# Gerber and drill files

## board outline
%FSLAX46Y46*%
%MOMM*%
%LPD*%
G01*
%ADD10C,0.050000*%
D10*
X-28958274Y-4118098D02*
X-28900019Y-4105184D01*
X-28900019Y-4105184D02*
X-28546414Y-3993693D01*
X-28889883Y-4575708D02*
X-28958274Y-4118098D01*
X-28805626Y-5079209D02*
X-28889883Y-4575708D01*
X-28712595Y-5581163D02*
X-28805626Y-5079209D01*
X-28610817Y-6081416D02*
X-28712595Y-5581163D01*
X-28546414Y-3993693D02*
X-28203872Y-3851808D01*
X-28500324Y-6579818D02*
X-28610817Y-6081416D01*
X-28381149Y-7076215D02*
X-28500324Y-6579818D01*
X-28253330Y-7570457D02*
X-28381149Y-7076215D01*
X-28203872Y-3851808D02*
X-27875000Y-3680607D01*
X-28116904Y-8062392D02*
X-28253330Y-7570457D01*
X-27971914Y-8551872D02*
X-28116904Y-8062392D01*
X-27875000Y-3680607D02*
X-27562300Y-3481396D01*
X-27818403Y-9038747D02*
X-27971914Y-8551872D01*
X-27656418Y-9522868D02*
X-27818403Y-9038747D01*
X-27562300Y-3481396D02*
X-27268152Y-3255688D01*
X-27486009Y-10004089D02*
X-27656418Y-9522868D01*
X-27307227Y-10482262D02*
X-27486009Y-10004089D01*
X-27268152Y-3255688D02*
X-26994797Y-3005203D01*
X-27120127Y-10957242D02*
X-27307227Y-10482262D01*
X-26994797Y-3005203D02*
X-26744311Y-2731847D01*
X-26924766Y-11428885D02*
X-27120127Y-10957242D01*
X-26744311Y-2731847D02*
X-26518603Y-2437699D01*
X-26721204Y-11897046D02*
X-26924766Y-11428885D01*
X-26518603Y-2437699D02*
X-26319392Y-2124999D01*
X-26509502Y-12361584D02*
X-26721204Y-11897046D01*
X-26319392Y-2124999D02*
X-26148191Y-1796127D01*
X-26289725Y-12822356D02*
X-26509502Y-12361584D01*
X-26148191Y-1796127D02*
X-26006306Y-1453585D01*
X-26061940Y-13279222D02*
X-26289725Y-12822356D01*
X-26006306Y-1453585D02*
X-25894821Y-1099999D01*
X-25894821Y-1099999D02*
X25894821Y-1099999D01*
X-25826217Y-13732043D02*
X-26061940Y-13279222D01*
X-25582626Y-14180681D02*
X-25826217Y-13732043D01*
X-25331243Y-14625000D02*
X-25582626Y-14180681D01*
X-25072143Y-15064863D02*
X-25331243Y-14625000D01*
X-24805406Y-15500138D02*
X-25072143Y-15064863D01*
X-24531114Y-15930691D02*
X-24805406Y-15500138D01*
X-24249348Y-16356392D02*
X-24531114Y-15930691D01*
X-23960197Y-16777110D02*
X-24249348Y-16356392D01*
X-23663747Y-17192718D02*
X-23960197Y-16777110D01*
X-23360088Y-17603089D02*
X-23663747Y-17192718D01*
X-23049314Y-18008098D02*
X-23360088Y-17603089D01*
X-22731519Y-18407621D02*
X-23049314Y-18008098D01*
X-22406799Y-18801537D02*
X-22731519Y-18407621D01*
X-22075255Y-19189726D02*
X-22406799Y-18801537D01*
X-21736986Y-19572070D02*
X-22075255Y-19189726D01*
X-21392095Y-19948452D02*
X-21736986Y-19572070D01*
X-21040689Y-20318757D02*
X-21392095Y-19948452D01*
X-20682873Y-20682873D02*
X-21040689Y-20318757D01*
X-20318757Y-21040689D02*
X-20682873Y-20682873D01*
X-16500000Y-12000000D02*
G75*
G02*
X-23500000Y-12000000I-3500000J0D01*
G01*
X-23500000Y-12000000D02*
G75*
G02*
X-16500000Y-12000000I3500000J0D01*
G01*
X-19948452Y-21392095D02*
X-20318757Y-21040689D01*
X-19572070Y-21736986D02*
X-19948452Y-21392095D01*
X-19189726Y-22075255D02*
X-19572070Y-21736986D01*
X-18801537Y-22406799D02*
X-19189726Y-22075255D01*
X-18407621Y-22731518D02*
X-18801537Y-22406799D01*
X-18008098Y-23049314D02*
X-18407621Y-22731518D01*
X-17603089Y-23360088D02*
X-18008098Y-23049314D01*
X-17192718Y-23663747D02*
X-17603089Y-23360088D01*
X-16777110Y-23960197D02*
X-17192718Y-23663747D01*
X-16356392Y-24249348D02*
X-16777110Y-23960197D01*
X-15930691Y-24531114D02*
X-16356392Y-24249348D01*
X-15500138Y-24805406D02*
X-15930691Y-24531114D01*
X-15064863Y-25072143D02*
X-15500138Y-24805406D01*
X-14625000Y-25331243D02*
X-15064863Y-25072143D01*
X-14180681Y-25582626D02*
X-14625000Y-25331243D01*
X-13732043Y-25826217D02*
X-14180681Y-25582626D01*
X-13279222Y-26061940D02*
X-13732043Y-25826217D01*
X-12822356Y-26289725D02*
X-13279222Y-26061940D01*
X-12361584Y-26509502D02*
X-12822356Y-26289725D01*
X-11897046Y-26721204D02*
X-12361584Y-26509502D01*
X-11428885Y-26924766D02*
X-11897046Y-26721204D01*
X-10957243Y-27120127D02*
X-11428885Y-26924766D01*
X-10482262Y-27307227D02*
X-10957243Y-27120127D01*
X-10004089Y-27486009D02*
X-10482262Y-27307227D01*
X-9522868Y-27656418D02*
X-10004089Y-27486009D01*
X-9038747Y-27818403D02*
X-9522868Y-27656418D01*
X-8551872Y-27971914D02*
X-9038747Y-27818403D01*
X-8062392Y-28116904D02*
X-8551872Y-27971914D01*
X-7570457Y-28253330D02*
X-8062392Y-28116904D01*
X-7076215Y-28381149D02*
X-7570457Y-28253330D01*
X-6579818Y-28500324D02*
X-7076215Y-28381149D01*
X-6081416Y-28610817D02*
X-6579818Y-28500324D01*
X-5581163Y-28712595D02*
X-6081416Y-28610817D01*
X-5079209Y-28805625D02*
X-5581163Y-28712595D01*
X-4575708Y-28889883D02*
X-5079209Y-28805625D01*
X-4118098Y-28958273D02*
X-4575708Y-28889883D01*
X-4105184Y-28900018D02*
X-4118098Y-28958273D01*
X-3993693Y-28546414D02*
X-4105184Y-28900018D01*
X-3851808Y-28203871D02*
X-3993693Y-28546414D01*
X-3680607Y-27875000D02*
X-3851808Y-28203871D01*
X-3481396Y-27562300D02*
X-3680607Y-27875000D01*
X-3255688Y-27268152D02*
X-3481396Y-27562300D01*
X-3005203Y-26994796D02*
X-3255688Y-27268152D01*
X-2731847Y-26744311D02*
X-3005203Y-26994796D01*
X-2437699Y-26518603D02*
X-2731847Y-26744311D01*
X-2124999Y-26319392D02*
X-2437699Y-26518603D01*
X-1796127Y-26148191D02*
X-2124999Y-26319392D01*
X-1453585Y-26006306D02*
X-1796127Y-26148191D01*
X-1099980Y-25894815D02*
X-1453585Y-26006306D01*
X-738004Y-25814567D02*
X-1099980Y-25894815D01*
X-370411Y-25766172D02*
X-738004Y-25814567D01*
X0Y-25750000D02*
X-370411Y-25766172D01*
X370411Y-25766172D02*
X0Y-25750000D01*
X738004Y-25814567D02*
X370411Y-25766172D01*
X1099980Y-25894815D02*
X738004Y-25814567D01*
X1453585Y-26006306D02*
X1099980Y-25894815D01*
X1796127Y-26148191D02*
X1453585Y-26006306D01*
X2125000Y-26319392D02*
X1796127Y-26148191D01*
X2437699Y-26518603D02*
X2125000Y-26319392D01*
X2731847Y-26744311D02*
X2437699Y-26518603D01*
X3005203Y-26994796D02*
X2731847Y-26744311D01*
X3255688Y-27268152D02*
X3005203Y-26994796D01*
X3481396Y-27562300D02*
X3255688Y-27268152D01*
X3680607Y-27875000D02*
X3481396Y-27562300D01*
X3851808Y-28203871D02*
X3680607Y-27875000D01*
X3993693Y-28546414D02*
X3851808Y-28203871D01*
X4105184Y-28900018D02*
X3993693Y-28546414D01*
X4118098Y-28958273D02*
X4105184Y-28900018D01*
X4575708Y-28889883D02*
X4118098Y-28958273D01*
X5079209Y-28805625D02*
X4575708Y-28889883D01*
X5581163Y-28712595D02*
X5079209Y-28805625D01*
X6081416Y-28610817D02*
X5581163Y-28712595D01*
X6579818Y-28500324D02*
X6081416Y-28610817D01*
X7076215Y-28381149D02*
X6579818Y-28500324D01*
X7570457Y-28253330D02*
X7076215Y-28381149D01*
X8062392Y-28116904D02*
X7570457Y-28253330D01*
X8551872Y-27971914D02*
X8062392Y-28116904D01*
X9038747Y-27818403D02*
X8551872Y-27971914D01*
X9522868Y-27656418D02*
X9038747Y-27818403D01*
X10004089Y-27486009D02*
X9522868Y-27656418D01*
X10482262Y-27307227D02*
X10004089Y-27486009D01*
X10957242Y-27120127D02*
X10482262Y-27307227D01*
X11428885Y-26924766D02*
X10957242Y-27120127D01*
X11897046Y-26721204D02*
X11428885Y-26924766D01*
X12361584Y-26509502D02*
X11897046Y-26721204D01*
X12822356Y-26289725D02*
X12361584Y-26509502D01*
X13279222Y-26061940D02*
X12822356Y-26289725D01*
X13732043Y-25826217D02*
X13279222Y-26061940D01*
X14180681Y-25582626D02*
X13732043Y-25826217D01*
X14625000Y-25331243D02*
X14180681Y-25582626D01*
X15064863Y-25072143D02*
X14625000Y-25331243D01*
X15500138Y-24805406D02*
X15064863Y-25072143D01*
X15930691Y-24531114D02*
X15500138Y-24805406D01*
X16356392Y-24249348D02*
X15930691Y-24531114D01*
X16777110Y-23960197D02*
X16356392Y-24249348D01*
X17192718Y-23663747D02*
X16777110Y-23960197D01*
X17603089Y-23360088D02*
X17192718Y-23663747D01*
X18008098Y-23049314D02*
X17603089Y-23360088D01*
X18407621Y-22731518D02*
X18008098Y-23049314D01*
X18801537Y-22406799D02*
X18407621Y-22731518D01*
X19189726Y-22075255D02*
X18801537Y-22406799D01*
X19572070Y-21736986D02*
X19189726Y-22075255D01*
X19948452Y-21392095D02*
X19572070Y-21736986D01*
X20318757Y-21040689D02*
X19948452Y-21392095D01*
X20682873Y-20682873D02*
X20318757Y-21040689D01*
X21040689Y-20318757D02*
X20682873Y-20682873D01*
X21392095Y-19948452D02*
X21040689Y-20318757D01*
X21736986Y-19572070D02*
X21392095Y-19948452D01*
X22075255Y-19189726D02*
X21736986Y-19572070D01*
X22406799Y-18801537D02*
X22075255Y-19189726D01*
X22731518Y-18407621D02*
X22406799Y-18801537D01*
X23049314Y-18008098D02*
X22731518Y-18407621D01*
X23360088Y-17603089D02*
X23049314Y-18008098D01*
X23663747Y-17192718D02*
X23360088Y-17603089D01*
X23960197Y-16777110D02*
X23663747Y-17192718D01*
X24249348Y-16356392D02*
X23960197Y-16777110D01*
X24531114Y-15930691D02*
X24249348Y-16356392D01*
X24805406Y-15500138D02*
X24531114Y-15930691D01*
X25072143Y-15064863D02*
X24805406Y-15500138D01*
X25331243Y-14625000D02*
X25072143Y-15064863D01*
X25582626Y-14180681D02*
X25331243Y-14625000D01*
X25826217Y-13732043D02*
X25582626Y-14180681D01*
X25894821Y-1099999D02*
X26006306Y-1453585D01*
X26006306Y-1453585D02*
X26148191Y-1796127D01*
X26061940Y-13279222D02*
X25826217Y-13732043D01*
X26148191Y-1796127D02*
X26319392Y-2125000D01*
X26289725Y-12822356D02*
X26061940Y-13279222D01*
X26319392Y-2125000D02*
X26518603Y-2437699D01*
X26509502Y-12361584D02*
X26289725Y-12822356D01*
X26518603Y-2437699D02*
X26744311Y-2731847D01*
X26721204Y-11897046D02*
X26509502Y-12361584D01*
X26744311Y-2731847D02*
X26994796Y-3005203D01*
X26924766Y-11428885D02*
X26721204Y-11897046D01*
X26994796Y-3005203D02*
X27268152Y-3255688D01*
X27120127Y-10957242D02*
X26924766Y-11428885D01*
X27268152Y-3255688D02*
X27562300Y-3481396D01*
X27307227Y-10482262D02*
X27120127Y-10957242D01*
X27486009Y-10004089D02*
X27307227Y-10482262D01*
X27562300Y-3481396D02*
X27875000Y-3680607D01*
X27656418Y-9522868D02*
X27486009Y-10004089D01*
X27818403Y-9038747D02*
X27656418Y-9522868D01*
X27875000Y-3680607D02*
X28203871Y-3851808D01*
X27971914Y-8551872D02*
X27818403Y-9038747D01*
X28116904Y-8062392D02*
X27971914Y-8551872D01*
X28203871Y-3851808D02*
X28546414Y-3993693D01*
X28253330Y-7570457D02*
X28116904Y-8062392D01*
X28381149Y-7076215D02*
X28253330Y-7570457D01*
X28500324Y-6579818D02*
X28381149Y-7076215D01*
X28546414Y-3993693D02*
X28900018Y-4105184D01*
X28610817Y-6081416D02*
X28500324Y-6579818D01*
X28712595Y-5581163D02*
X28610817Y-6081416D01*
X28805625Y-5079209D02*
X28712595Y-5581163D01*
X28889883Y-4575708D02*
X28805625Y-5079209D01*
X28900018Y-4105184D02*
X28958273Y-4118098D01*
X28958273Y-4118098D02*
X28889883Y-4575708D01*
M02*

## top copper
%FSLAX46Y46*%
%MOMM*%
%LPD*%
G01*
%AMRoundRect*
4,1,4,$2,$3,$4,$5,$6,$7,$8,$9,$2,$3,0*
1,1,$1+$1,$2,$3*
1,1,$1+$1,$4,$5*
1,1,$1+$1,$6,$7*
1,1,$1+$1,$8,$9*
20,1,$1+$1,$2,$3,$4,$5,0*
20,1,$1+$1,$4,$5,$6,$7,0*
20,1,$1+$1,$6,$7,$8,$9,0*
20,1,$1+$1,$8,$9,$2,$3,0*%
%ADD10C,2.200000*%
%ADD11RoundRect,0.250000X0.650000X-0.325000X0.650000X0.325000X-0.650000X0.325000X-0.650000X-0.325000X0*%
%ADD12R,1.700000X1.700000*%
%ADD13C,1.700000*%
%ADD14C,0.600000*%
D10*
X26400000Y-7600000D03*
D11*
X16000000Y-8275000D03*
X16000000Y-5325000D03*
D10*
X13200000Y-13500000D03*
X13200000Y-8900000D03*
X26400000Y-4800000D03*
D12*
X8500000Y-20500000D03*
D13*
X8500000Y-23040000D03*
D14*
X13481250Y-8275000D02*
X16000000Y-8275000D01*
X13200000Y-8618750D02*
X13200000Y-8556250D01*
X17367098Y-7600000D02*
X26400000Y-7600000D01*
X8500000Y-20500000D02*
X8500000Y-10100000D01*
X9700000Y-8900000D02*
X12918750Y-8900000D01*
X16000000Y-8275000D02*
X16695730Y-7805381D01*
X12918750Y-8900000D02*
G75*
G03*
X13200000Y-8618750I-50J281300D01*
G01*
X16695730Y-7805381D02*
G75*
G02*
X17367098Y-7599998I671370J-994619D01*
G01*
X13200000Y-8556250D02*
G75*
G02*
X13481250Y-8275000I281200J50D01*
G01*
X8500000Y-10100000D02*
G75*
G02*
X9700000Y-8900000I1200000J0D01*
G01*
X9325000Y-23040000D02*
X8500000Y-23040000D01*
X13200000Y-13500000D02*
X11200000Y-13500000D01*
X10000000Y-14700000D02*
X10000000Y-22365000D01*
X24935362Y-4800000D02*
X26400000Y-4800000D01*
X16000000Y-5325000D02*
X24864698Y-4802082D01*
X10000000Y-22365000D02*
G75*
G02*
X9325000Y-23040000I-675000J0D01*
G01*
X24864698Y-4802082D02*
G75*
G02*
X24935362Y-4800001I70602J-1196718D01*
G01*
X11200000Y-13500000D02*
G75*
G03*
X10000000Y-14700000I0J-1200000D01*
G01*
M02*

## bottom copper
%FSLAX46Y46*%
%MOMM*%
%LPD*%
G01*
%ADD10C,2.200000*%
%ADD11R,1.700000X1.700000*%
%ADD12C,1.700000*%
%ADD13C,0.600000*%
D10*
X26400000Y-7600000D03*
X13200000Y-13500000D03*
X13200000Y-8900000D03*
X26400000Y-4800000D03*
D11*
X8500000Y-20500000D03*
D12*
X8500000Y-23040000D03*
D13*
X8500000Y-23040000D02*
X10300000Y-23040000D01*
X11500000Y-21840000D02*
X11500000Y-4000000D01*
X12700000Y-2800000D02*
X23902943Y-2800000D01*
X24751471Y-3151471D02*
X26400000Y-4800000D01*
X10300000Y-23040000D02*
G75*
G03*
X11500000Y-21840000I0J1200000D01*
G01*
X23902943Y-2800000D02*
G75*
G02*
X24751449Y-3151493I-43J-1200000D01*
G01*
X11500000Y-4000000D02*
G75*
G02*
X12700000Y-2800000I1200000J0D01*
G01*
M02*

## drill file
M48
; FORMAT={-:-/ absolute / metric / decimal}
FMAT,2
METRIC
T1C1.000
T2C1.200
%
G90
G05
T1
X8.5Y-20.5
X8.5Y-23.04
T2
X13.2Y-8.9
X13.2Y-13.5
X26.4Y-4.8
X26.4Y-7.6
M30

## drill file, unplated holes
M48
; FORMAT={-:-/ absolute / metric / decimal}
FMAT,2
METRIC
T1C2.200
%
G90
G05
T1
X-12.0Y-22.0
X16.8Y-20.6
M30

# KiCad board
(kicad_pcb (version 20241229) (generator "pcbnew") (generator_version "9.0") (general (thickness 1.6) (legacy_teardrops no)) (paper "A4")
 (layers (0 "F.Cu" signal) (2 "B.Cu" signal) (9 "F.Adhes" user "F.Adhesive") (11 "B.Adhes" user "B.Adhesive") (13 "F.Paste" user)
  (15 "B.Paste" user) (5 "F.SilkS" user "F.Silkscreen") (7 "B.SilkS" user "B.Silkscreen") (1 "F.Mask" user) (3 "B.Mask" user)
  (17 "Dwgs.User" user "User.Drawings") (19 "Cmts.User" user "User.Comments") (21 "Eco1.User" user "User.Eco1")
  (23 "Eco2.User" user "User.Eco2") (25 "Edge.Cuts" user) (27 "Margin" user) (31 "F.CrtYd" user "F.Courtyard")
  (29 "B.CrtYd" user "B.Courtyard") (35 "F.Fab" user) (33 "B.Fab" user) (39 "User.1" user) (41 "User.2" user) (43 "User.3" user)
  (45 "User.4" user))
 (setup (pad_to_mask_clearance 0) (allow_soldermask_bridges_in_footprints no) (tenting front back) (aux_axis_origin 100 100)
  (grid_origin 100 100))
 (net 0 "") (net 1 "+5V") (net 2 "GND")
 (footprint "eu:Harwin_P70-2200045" (layer "F.Cu") (at 126.4 107.6)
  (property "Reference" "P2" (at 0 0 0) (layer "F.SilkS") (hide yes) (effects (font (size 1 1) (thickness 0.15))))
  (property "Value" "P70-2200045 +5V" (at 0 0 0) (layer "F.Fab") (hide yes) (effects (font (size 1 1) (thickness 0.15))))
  (pad "1" thru_hole circle (at 0 0) (size 2.2 2.2) (drill 1.2) (layers "*.Cu" "*.Mask" "F.Paste") (remove_unused_layers no) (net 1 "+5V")))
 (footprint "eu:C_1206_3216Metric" (layer "F.Cu") (at 116 106.8 90)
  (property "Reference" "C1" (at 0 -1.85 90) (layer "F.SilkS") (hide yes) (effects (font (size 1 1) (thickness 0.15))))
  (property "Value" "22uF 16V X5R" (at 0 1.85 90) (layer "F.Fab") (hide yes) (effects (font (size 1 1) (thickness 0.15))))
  (pad "1" smd roundrect (at -1.475 0 90) (size 1.15 1.8) (layers "F.Cu" "F.Mask" "F.Paste") (roundrect_rratio 0.217391) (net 1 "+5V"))
  (pad "2" smd roundrect (at 1.475 0 90) (size 1.15 1.8) (layers "F.Cu" "F.Mask" "F.Paste") (roundrect_rratio 0.217391) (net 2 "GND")))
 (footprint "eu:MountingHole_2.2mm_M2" (layer "F.Cu") (at 88 122)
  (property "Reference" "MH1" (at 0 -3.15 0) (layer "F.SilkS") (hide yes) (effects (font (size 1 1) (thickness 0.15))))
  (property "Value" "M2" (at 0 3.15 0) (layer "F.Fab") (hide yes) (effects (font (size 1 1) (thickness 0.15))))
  (pad "" np_thru_hole circle (at 0 0) (size 2.2 2.2) (drill 2.2) (layers "*.Cu" "*.Mask")))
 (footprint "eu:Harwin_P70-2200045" (layer "F.Cu") (at 113.2 113.5)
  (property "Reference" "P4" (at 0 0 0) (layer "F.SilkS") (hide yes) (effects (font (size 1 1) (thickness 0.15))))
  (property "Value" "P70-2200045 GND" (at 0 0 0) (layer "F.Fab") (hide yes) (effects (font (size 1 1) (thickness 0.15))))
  (pad "1" thru_hole circle (at 0 0) (size 2.2 2.2) (drill 1.2) (layers "*.Cu" "*.Mask" "F.Paste") (remove_unused_layers no) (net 2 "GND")))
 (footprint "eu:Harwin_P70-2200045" (layer "F.Cu") (at 113.2 108.9)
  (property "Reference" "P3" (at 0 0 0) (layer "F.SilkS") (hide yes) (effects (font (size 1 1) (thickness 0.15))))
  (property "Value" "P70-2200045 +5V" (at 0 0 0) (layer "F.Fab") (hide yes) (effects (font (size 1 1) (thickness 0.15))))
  (pad "1" thru_hole circle (at 0 0) (size 2.2 2.2) (drill 1.2) (layers "*.Cu" "*.Mask" "F.Paste") (remove_unused_layers no) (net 1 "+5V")))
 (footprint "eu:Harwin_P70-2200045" (layer "F.Cu") (at 126.4 104.8)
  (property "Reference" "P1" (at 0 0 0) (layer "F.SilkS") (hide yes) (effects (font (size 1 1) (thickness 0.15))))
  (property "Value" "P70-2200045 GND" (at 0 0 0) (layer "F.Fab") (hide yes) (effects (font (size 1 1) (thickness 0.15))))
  (pad "1" thru_hole circle (at 0 0) (size 2.2 2.2) (drill 1.2) (layers "*.Cu" "*.Mask" "F.Paste") (remove_unused_layers no) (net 2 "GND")))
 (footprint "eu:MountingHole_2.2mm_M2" (layer "F.Cu") (at 116.8 120.6)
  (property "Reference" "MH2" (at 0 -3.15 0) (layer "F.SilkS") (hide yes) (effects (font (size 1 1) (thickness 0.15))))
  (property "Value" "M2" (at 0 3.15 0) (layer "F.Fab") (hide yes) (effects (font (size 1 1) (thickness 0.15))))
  (pad "" np_thru_hole circle (at 0 0) (size 2.2 2.2) (drill 2.2) (layers "*.Cu" "*.Mask")))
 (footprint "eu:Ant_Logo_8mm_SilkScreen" (layer "B.Cu") (at 90.1 106.7 180)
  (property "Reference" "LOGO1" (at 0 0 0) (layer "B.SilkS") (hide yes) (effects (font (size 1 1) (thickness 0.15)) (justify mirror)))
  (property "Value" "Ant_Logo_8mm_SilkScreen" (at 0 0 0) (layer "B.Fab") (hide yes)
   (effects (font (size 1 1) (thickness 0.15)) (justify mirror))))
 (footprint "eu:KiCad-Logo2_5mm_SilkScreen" (layer "B.Cu") (at 102.4 105.7 180)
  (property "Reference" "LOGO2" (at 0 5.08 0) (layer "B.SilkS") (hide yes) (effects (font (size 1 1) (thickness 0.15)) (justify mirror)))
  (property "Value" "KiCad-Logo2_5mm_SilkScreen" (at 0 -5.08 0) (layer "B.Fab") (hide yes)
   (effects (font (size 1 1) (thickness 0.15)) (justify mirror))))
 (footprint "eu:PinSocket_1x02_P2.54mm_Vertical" (layer "B.Cu") (at 108.5 120.5 180)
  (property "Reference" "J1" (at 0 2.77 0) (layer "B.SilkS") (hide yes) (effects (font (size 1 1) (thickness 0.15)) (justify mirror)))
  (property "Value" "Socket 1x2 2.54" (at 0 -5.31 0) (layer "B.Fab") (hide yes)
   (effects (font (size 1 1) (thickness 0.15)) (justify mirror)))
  (pad "1" thru_hole rect (at 0 0 180) (size 1.7 1.7) (drill 1) (layers "*.Cu" "*.Mask") (remove_unused_layers no) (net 1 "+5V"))
  (pad "2" thru_hole circle (at 0 -2.54 180) (size 1.7 1.7) (drill 1) (layers "*.Cu" "*.Mask") (remove_unused_layers no) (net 2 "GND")))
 (gr_line (start 71.041726 104.118098) (end 71.099981 104.105184) (stroke (width 0.05) (type default)) (layer "Edge.Cuts"))
 (gr_line (start 71.099981 104.105184) (end 71.453586 103.993693) (stroke (width 0.05) (type default)) (layer "Edge.Cuts"))
 (gr_line (start 71.110117 104.575708) (end 71.041726 104.118098) (stroke (width 0.05) (type default)) (layer "Edge.Cuts"))
 (gr_line (start 71.194374 105.079209) (end 71.110117 104.575708) (stroke (width 0.05) (type default)) (layer "Edge.Cuts"))
 (gr_line (start 71.287405 105.581163) (end 71.194374 105.079209) (stroke (width 0.05) (type default)) (layer "Edge.Cuts"))
 (gr_line (start 71.389183 106.081416) (end 71.287405 105.581163) (stroke (width 0.05) (type default)) (layer "Edge.Cuts"))
 (gr_line (start 71.453586 103.993693) (end 71.796128 103.851808) (stroke (width 0.05) (type default)) (layer "Edge.Cuts"))
 (gr_line (start 71.499676 106.579818) (end 71.389183 106.081416) (stroke (width 0.05) (type default)) (layer "Edge.Cuts"))
 (gr_line (start 71.618851 107.076215) (end 71.499676 106.579818) (stroke (width 0.05) (type default)) (layer "Edge.Cuts"))
 (gr_line (start 71.74667 107.570457) (end 71.618851 107.076215) (stroke (width 0.05) (type default)) (layer "Edge.Cuts"))
 (gr_line (start 71.796128 103.851808) (end 72.125 103.680607) (stroke (width 0.05) (type default)) (layer "Edge.Cuts"))
 (gr_line (start 71.883096 108.062392) (end 71.74667 107.570457) (stroke (width 0.05) (type default)) (layer "Edge.Cuts"))
 (gr_line (start 72.028086 108.551872) (end 71.883096 108.062392) (stroke (width 0.05) (type default)) (layer "Edge.Cuts"))
 (gr_line (start 72.125 103.680607) (end 72.4377 103.481396) (stroke (width 0.05) (type default)) (layer "Edge.Cuts"))
 (gr_line (start 72.181597 109.038747) (end 72.028086 108.551872) (stroke (width 0.05) (type default)) (layer "Edge.Cuts"))
 (gr_line (start 72.343582 109.522868) (end 72.181597 109.038747) (stroke (width 0.05) (type default)) (layer "Edge.Cuts"))
 (gr_line (start 72.4377 103.481396) (end 72.731848 103.255688) (stroke (width 0.05) (type default)) (layer "Edge.Cuts"))
 (gr_line (start 72.513991 110.004089) (end 72.343582 109.522868) (stroke (width 0.05) (type default)) (layer "Edge.Cuts"))
 (gr_line (start 72.692773 110.482262) (end 72.513991 110.004089) (stroke (width 0.05) (type default)) (layer "Edge.Cuts"))
 (gr_line (start 72.731848 103.255688) (end 73.005203 103.005203) (stroke (width 0.05) (type default)) (layer "Edge.Cuts"))
 (gr_line (start 72.879873 110.957242) (end 72.692773 110.482262) (stroke (width 0.05) (type default)) (layer "Edge.Cuts"))
 (gr_line (start 73.005203 103.005203) (end 73.255689 102.731847) (stroke (width 0.05) (type default)) (layer "Edge.Cuts"))
 (gr_line (start 73.075234 111.428885) (end 72.879873 110.957242) (stroke (width 0.05) (type default)) (layer "Edge.Cuts"))
 (gr_line (start 73.255689 102.731847) (end 73.481397 102.437699) (stroke (width 0.05) (type default)) (layer "Edge.Cuts"))
 (gr_line (start 73.278796 111.897046) (end 73.075234 111.428885) (stroke (width 0.05) (type default)) (layer "Edge.Cuts"))
 (gr_line (start 73.481397 102.437699) (end 73.680608 102.124999) (stroke (width 0.05) (type default)) (layer "Edge.Cuts"))
 (gr_line (start 73.490498 112.361584) (end 73.278796 111.897046) (stroke (width 0.05) (type default)) (layer "Edge.Cuts"))
 (gr_line (start 73.680608 102.124999) (end 73.851809 101.796127) (stroke (width 0.05) (type default)) (layer "Edge.Cuts"))
 (gr_line (start 73.710275 112.822356) (end 73.490498 112.361584) (stroke (width 0.05) (type default)) (layer "Edge.Cuts"))
 (gr_line (start 73.851809 101.796127) (end 73.993694 101.453585) (stroke (width 0.05) (type default)) (layer "Edge.Cuts"))
 (gr_line (start 73.93806 113.279222) (end 73.710275 112.822356) (stroke (width 0.05) (type default)) (layer "Edge.Cuts"))
 (gr_line (start 73.993694 101.453585) (end 74.105179 101.099999) (stroke (width 0.05) (type default)) (layer "Edge.Cuts"))
 (gr_line (start 74.105179 101.099999) (end 125.894821 101.099999) (stroke (width 0.05) (type default)) (layer "Edge.Cuts"))
 (gr_line (start 74.173783 113.732043) (end 73.93806 113.279222) (stroke (width 0.05) (type default)) (layer "Edge.Cuts"))
 (gr_line (start 74.417374 114.180681) (end 74.173783 113.732043) (stroke (width 0.05) (type default)) (layer "Edge.Cuts"))
 (gr_line (start 74.668757 114.625) (end 74.417374 114.180681) (stroke (width 0.05) (type default)) (layer "Edge.Cuts"))
 (gr_line (start 74.927857 115.064863) (end 74.668757 114.625) (stroke (width 0.05) (type default)) (layer "Edge.Cuts"))
 (gr_line (start 75.194594 115.500138) (end 74.927857 115.064863) (stroke (width 0.05) (type default)) (layer "Edge.Cuts"))
 (gr_line (start 75.468886 115.930691) (end 75.194594 115.500138) (stroke (width 0.05) (type default)) (layer "Edge.Cuts"))
 (gr_line (start 75.750652 116.356392) (end 75.468886 115.930691) (stroke (width 0.05) (type default)) (layer "Edge.Cuts"))
 (gr_line (start 76.039803 116.77711) (end 75.750652 116.356392) (stroke (width 0.05) (type default)) (layer "Edge.Cuts"))
 (gr_line (start 76.336253 117.192718) (end 76.039803 116.77711) (stroke (width 0.05) (type default)) (layer "Edge.Cuts"))
 (gr_line (start 76.639912 117.603089) (end 76.336253 117.192718) (stroke (width 0.05) (type default)) (layer "Edge.Cuts"))
 (gr_line (start 76.950686 118.008098) (end 76.639912 117.603089) (stroke (width 0.05) (type default)) (layer "Edge.Cuts"))
 (gr_line (start 77.268481 118.407621) (end 76.950686 118.008098) (stroke (width 0.05) (type default)) (layer "Edge.Cuts"))
 (gr_line (start 77.593201 118.801537) (end 77.268481 118.407621) (stroke (width 0.05) (type default)) (layer "Edge.Cuts"))
 (gr_line (start 77.924745 119.189726) (end 77.593201 118.801537) (stroke (width 0.05) (type default)) (layer "Edge.Cuts"))
 (gr_line (start 78.263014 119.57207) (end 77.924745 119.189726) (stroke (width 0.05) (type default)) (layer "Edge.Cuts"))
 (gr_line (start 78.607905 119.948452) (end 78.263014 119.57207) (stroke (width 0.05) (type default)) (layer "Edge.Cuts"))
 (gr_line (start 78.959311 120.318757) (end 78.607905 119.948452) (stroke (width 0.05) (type default)) (layer "Edge.Cuts"))
 (gr_line (start 79.317127 120.682873) (end 78.959311 120.318757) (stroke (width 0.05) (type default)) (layer "Edge.Cuts"))
 (gr_line (start 79.681243 121.040689) (end 79.317127 120.682873) (stroke (width 0.05) (type default)) (layer "Edge.Cuts"))
 (gr_circle (center 80 112) (end 83.5 112) (stroke (width 0.05) (type default)) (fill no) (layer "Edge.Cuts"))
 (gr_line (start 80.051548 121.392095) (end 79.681243 121.040689) (stroke (width 0.05) (type default)) (layer "Edge.Cuts"))
 (gr_line (start 80.42793 121.736986) (end 80.051548 121.392095) (stroke (width 0.05) (type default)) (layer "Edge.Cuts"))
 (gr_line (start 80.810274 122.075255) (end 80.42793 121.736986) (stroke (width 0.05) (type default)) (layer "Edge.Cuts"))
 (gr_line (start 81.198463 122.406799) (end 80.810274 122.075255) (stroke (width 0.05) (type default)) (layer "Edge.Cuts"))
 (gr_line (start 81.592379 122.731518) (end 81.198463 122.406799) (stroke (width 0.05) (type default)) (layer "Edge.Cuts"))
 (gr_line (start 81.991902 123.049314) (end 81.592379 122.731518) (stroke (width 0.05) (type default)) (layer "Edge.Cuts"))
 (gr_line (start 82.396911 123.360088) (end 81.991902 123.049314) (stroke (width 0.05) (type default)) (layer "Edge.Cuts"))
 (gr_line (start 82.807282 123.663747) (end 82.396911 123.360088) (stroke (width 0.05) (type default)) (layer "Edge.Cuts"))
 (gr_line (start 83.22289 123.960197) (end 82.807282 123.663747) (stroke (width 0.05) (type default)) (layer "Edge.Cuts"))
 (gr_line (start 83.643608 124.249348) (end 83.22289 123.960197) (stroke (width 0.05) (type default)) (layer "Edge.Cuts"))
 (gr_line (start 84.069309 124.531114) (end 83.643608 124.249348) (stroke (width 0.05) (type default)) (layer "Edge.Cuts"))
 (gr_line (start 84.499862 124.805406) (end 84.069309 124.531114) (stroke (width 0.05) (type default)) (layer "Edge.Cuts"))
 (gr_line (start 84.935137 125.072143) (end 84.499862 124.805406) (stroke (width 0.05) (type default)) (layer "Edge.Cuts"))
 (gr_line (start 85.375 125.331243) (end 84.935137 125.072143) (stroke (width 0.05) (type default)) (layer "Edge.Cuts"))
 (gr_line (start 85.819319 125.582626) (end 85.375 125.331243) (stroke (width 0.05) (type default)) (layer "Edge.Cuts"))
 (gr_line (start 86.267957 125.826217) (end 85.819319 125.582626) (stroke (width 0.05) (type default)) (layer "Edge.Cuts"))
 (gr_line (start 86.720778 126.06194) (end 86.267957 125.826217) (stroke (width 0.05) (type default)) (layer "Edge.Cuts"))
 (gr_line (start 87.177644 126.289725) (end 86.720778 126.06194) (stroke (width 0.05) (type default)) (layer "Edge.Cuts"))
 (gr_line (start 87.638416 126.509502) (end 87.177644 126.289725) (stroke (width 0.05) (type default)) (layer "Edge.Cuts"))
 (gr_line (start 88.102954 126.721204) (end 87.638416 126.509502) (stroke (width 0.05) (type default)) (layer "Edge.Cuts"))
 (gr_line (start 88.571115 126.924766) (end 88.102954 126.721204) (stroke (width 0.05) (type default)) (layer "Edge.Cuts"))
 (gr_line (start 89.042757 127.120127) (end 88.571115 126.924766) (stroke (width 0.05) (type default)) (layer "Edge.Cuts"))
 (gr_line (start 89.517738 127.307227) (end 89.042757 127.120127) (stroke (width 0.05) (type default)) (layer "Edge.Cuts"))
 (gr_line (start 89.995911 127.486009) (end 89.517738 127.307227) (stroke (width 0.05) (type default)) (layer "Edge.Cuts"))
 (gr_line (start 90.477132 127.656418) (end 89.995911 127.486009) (stroke (width 0.05) (type default)) (layer "Edge.Cuts"))
 (gr_line (start 90.961253 127.818403) (end 90.477132 127.656418) (stroke (width 0.05) (type default)) (layer "Edge.Cuts"))
 (gr_line (start 91.448128 127.971914) (end 90.961253 127.818403) (stroke (width 0.05) (type default)) (layer "Edge.Cuts"))
 (gr_line (start 91.937608 128.116904) (end 91.448128 127.971914) (stroke (width 0.05) (type default)) (layer "Edge.Cuts"))
 (gr_line (start 92.429543 128.25333) (end 91.937608 128.116904) (stroke (width 0.05) (type default)) (layer "Edge.Cuts"))
 (gr_line (start 92.923785 128.381149) (end 92.429543 128.25333) (stroke (width 0.05) (type default)) (layer "Edge.Cuts"))
 (gr_line (start 93.420182 128.500324) (end 92.923785 128.381149) (stroke (width 0.05) (type default)) (layer "Edge.Cuts"))
 (gr_line (start 93.918584 128.610817) (end 93.420182 128.500324) (stroke (width 0.05) (type default)) (layer "Edge.Cuts"))
 (gr_line (start 94.418837 128.712595) (end 93.918584 128.610817) (stroke (width 0.05) (type default)) (layer "Edge.Cuts"))
 (gr_line (start 94.920791 128.805625) (end 94.418837 128.712595) (stroke (width 0.05) (type default)) (layer "Edge.Cuts"))
 (gr_line (start 95.424292 128.889883) (end 94.920791 128.805625) (stroke (width 0.05) (type default)) (layer "Edge.Cuts"))
 (gr_line (start 95.881902 128.958273) (end 95.424292 128.889883) (stroke (width 0.05) (type default)) (layer "Edge.Cuts"))
 (gr_line (start 95.894816 128.900018) (end 95.881902 128.958273) (stroke (width 0.05) (type default)) (layer "Edge.Cuts"))
 (gr_line (start 96.006307 128.546414) (end 95.894816 128.900018) (stroke (width 0.05) (type default)) (layer "Edge.Cuts"))
 (gr_line (start 96.148192 128.203871) (end 96.006307 128.546414) (stroke (width 0.05) (type default)) (layer "Edge.Cuts"))
 (gr_line (start 96.319393 127.875) (end 96.148192 128.203871) (stroke (width 0.05) (type default)) (layer "Edge.Cuts"))
 (gr_line (start 96.518604 127.5623) (end 96.319393 127.875) (stroke (width 0.05) (type default)) (layer "Edge.Cuts"))
 (gr_line (start 96.744312 127.268152) (end 96.518604 127.5623) (stroke (width 0.05) (type default)) (layer "Edge.Cuts"))
 (gr_line (start 96.994797 126.994796) (end 96.744312 127.268152) (stroke (width 0.05) (type default)) (layer "Edge.Cuts"))
 (gr_line (start 97.268153 126.744311) (end 96.994797 126.994796) (stroke (width 0.05) (type default)) (layer "Edge.Cuts"))
 (gr_line (start 97.562301 126.518603) (end 97.268153 126.744311) (stroke (width 0.05) (type default)) (layer "Edge.Cuts"))
 (gr_line (start 97.875001 126.319392) (end 97.562301 126.518603) (stroke (width 0.05) (type default)) (layer "Edge.Cuts"))
 (gr_line (start 98.203873 126.148191) (end 97.875001 126.319392) (stroke (width 0.05) (type default)) (layer "Edge.Cuts"))
 (gr_line (start 98.546415 126.006306) (end 98.203873 126.148191) (stroke (width 0.05) (type default)) (layer "Edge.Cuts"))
 (gr_line (start 98.90002 125.894815) (end 98.546415 126.006306) (stroke (width 0.05) (type default)) (layer "Edge.Cuts"))
 (gr_line (start 99.261996 125.814567) (end 98.90002 125.894815) (stroke (width 0.05) (type default)) (layer "Edge.Cuts"))
 (gr_line (start 99.629589 125.766172) (end 99.261996 125.814567) (stroke (width 0.05) (type default)) (layer "Edge.Cuts"))
 (gr_line (start 100 125.75) (end 99.629589 125.766172) (stroke (width 0.05) (type default)) (layer "Edge.Cuts"))
 (gr_line (start 100.370411 125.766172) (end 100 125.75) (stroke (width 0.05) (type default)) (layer "Edge.Cuts"))
 (gr_line (start 100.738004 125.814567) (end 100.370411 125.766172) (stroke (width 0.05) (type default)) (layer "Edge.Cuts"))
 (gr_line (start 101.09998 125.894815) (end 100.738004 125.814567) (stroke (width 0.05) (type default)) (layer "Edge.Cuts"))
 (gr_line (start 101.453585 126.006306) (end 101.09998 125.894815) (stroke (width 0.05) (type default)) (layer "Edge.Cuts"))
 (gr_line (start 101.796127 126.148191) (end 101.453585 126.006306) (stroke (width 0.05) (type default)) (layer "Edge.Cuts"))
 (gr_line (start 102.125 126.319392) (end 101.796127 126.148191) (stroke (width 0.05) (type default)) (layer "Edge.Cuts"))
 (gr_line (start 102.437699 126.518603) (end 102.125 126.319392) (stroke (width 0.05) (type default)) (layer "Edge.Cuts"))
 (gr_line (start 102.731847 126.744311) (end 102.437699 126.518603) (stroke (width 0.05) (type default)) (layer "Edge.Cuts"))
 (gr_line (start 103.005203 126.994796) (end 102.731847 126.744311) (stroke (width 0.05) (type default)) (layer "Edge.Cuts"))
 (gr_line (start 103.255688 127.268152) (end 103.005203 126.994796) (stroke (width 0.05) (type default)) (layer "Edge.Cuts"))
 (gr_line (start 103.481396 127.5623) (end 103.255688 127.268152) (stroke (width 0.05) (type default)) (layer "Edge.Cuts"))
 (gr_line (start 103.680607 127.875) (end 103.481396 127.5623) (stroke (width 0.05) (type default)) (layer "Edge.Cuts"))
 (gr_line (start 103.851808 128.203871) (end 103.680607 127.875) (stroke (width 0.05) (type default)) (layer "Edge.Cuts"))
 (gr_line (start 103.993693 128.546414) (end 103.851808 128.203871) (stroke (width 0.05) (type default)) (layer "Edge.Cuts"))
 (gr_line (start 104.105184 128.900018) (end 103.993693 128.546414) (stroke (width 0.05) (type default)) (layer "Edge.Cuts"))
 (gr_line (start 104.118098 128.958273) (end 104.105184 128.900018) (stroke (width 0.05) (type default)) (layer "Edge.Cuts"))
 (gr_line (start 104.575708 128.889883) (end 104.118098 128.958273) (stroke (width 0.05) (type default)) (layer "Edge.Cuts"))
 (gr_line (start 105.079209 128.805625) (end 104.575708 128.889883) (stroke (width 0.05) (type default)) (layer "Edge.Cuts"))
 (gr_line (start 105.581163 128.712595) (end 105.079209 128.805625) (stroke (width 0.05) (type default)) (layer "Edge.Cuts"))
 (gr_line (start 106.081416 128.610817) (end 105.581163 128.712595) (stroke (width 0.05) (type default)) (layer "Edge.Cuts"))
 (gr_line (start 106.579818 128.500324) (end 106.081416 128.610817) (stroke (width 0.05) (type default)) (layer "Edge.Cuts"))
 (gr_line (start 107.076215 128.381149) (end 106.579818 128.500324) (stroke (width 0.05) (type default)) (layer "Edge.Cuts"))
 (gr_line (start 107.570457 128.25333) (end 107.076215 128.381149) (stroke (width 0.05) (type default)) (layer "Edge.Cuts"))
 (gr_line (start 108.062392 128.116904) (end 107.570457 128.25333) (stroke (width 0.05) (type default)) (layer "Edge.Cuts"))
 (gr_line (start 108.551872 127.971914) (end 108.062392 128.116904) (stroke (width 0.05) (type default)) (layer "Edge.Cuts"))
 (gr_line (start 109.038747 127.818403) (end 108.551872 127.971914) (stroke (width 0.05) (type default)) (layer "Edge.Cuts"))
 (gr_line (start 109.522868 127.656418) (end 109.038747 127.818403) (stroke (width 0.05) (type default)) (layer "Edge.Cuts"))
 (gr_line (start 110.004089 127.486009) (end 109.522868 127.656418) (stroke (width 0.05) (type default)) (layer "Edge.Cuts"))
 (gr_line (start 110.482262 127.307227) (end 110.004089 127.486009) (stroke (width 0.05) (type default)) (layer "Edge.Cuts"))
 (gr_line (start 110.957242 127.120127) (end 110.482262 127.307227) (stroke (width 0.05) (type default)) (layer "Edge.Cuts"))
 (gr_line (start 111.428885 126.924766) (end 110.957242 127.120127) (stroke (width 0.05) (type default)) (layer "Edge.Cuts"))
 (gr_line (start 111.897046 126.721204) (end 111.428885 126.924766) (stroke (width 0.05) (type default)) (layer "Edge.Cuts"))
 (gr_line (start 112.361584 126.509502) (end 111.897046 126.721204) (stroke (width 0.05) (type default)) (layer "Edge.Cuts"))
 (gr_line (start 112.822356 126.289725) (end 112.361584 126.509502) (stroke (width 0.05) (type default)) (layer "Edge.Cuts"))
 (gr_line (start 113.279222 126.06194) (end 112.822356 126.289725) (stroke (width 0.05) (type default)) (layer "Edge.Cuts"))
 (gr_line (start 113.732043 125.826217) (end 113.279222 126.06194) (stroke (width 0.05) (type default)) (layer "Edge.Cuts"))
 (gr_line (start 114.180681 125.582626) (end 113.732043 125.826217) (stroke (width 0.05) (type default)) (layer "Edge.Cuts"))
 (gr_line (start 114.625 125.331243) (end 114.180681 125.582626) (stroke (width 0.05) (type default)) (layer "Edge.Cuts"))
 (gr_line (start 115.064863 125.072143) (end 114.625 125.331243) (stroke (width 0.05) (type default)) (layer "Edge.Cuts"))
 (gr_line (start 115.500138 124.805406) (end 115.064863 125.072143) (stroke (width 0.05) (type default)) (layer "Edge.Cuts"))
 (gr_line (start 115.930691 124.531114) (end 115.500138 124.805406) (stroke (width 0.05) (type default)) (layer "Edge.Cuts"))
 (gr_line (start 116.356392 124.249348) (end 115.930691 124.531114) (stroke (width 0.05) (type default)) (layer "Edge.Cuts"))
 (gr_line (start 116.77711 123.960197) (end 116.356392 124.249348) (stroke (width 0.05) (type default)) (layer "Edge.Cuts"))
 (gr_line (start 117.192718 123.663747) (end 116.77711 123.960197) (stroke (width 0.05) (type default)) (layer "Edge.Cuts"))
 (gr_line (start 117.603089 123.360088) (end 117.192718 123.663747) (stroke (width 0.05) (type default)) (layer "Edge.Cuts"))
 (gr_line (start 118.008098 123.049314) (end 117.603089 123.360088) (stroke (width 0.05) (type default)) (layer "Edge.Cuts"))
 (gr_line (start 118.407621 122.731518) (end 118.008098 123.049314) (stroke (width 0.05) (type default)) (layer "Edge.Cuts"))
 (gr_line (start 118.801537 122.406799) (end 118.407621 122.731518) (stroke (width 0.05) (type default)) (layer "Edge.Cuts"))
 (gr_line (start 119.189726 122.075255) (end 118.801537 122.406799) (stroke (width 0.05) (type default)) (layer "Edge.Cuts"))
 (gr_line (start 119.57207 121.736986) (end 119.189726 122.075255) (stroke (width 0.05) (type default)) (layer "Edge.Cuts"))
 (gr_line (start 119.948452 121.392095) (end 119.57207 121.736986) (stroke (width 0.05) (type default)) (layer "Edge.Cuts"))
 (gr_line (start 120.318757 121.040689) (end 119.948452 121.392095) (stroke (width 0.05) (type default)) (layer "Edge.Cuts"))
 (gr_line (start 120.682873 120.682873) (end 120.318757 121.040689) (stroke (width 0.05) (type default)) (layer "Edge.Cuts"))
 (gr_line (start 121.040689 120.318757) (end 120.682873 120.682873) (stroke (width 0.05) (type default)) (layer "Edge.Cuts"))
 (gr_line (start 121.392095 119.948452) (end 121.040689 120.318757) (stroke (width 0.05) (type default)) (layer "Edge.Cuts"))
 (gr_line (start 121.736986 119.57207) (end 121.392095 119.948452) (stroke (width 0.05) (type default)) (layer "Edge.Cuts"))
 (gr_line (start 122.075255 119.189726) (end 121.736986 119.57207) (stroke (width 0.05) (type default)) (layer "Edge.Cuts"))
 (gr_line (start 122.406799 118.801537) (end 122.075255 119.189726) (stroke (width 0.05) (type default)) (layer "Edge.Cuts"))
 (gr_line (start 122.731518 118.407621) (end 122.406799 118.801537) (stroke (width 0.05) (type default)) (layer "Edge.Cuts"))
 (gr_line (start 123.049314 118.008098) (end 122.731518 118.407621) (stroke (width 0.05) (type default)) (layer "Edge.Cuts"))
 (gr_line (start 123.360088 117.603089) (end 123.049314 118.008098) (stroke (width 0.05) (type default)) (layer "Edge.Cuts"))
 (gr_line (start 123.663747 117.192718) (end 123.360088 117.603089) (stroke (width 0.05) (type default)) (layer "Edge.Cuts"))
 (gr_line (start 123.960197 116.77711) (end 123.663747 117.192718) (stroke (width 0.05) (type default)) (layer "Edge.Cuts"))
 (gr_line (start 124.249348 116.356392) (end 123.960197 116.77711) (stroke (width 0.05) (type default)) (layer "Edge.Cuts"))
 (gr_line (start 124.531114 115.930691) (end 124.249348 116.356392) (stroke (width 0.05) (type default)) (layer "Edge.Cuts"))
 (gr_line (start 124.805406 115.500138) (end 124.531114 115.930691) (stroke (width 0.05) (type default)) (layer "Edge.Cuts"))
 (gr_line (start 125.072143 115.064863) (end 124.805406 115.500138) (stroke (width 0.05) (type default)) (layer "Edge.Cuts"))
 (gr_line (start 125.331243 114.625) (end 125.072143 115.064863) (stroke (width 0.05) (type default)) (layer "Edge.Cuts"))
 (gr_line (start 125.582626 114.180681) (end 125.331243 114.625) (stroke (width 0.05) (type default)) (layer "Edge.Cuts"))
 (gr_line (start 125.826217 113.732043) (end 125.582626 114.180681) (stroke (width 0.05) (type default)) (layer "Edge.Cuts"))
 (gr_line (start 125.894821 101.099999) (end 126.006306 101.453585) (stroke (width 0.05) (type default)) (layer "Edge.Cuts"))
 (gr_line (start 126.006306 101.453585) (end 126.148191 101.796127) (stroke (width 0.05) (type default)) (layer "Edge.Cuts"))
 (gr_line (start 126.06194 113.279222) (end 125.826217 113.732043) (stroke (width 0.05) (type default)) (layer "Edge.Cuts"))
 (gr_line (start 126.148191 101.796127) (end 126.319392 102.125) (stroke (width 0.05) (type default)) (layer "Edge.Cuts"))
 (gr_line (start 126.289725 112.822356) (end 126.06194 113.279222) (stroke (width 0.05) (type default)) (layer "Edge.Cuts"))
 (gr_line (start 126.319392 102.125) (end 126.518603 102.437699) (stroke (width 0.05) (type default)) (layer "Edge.Cuts"))
 (gr_line (start 126.509502 112.361584) (end 126.289725 112.822356) (stroke (width 0.05) (type default)) (layer "Edge.Cuts"))
 (gr_line (start 126.518603 102.437699) (end 126.744311 102.731847) (stroke (width 0.05) (type default)) (layer "Edge.Cuts"))
 (gr_line (start 126.721204 111.897046) (end 126.509502 112.361584) (stroke (width 0.05) (type default)) (layer "Edge.Cuts"))
 (gr_line (start 126.744311 102.731847) (end 126.994796 103.005203) (stroke (width 0.05) (type default)) (layer "Edge.Cuts"))
 (gr_line (start 126.924766 111.428885) (end 126.721204 111.897046) (stroke (width 0.05) (type default)) (layer "Edge.Cuts"))
 (gr_line (start 126.994796 103.005203) (end 127.268152 103.255688) (stroke (width 0.05) (type default)) (layer "Edge.Cuts"))
 (gr_line (start 127.120127 110.957242) (end 126.924766 111.428885) (stroke (width 0.05) (type default)) (layer "Edge.Cuts"))
 (gr_line (start 127.268152 103.255688) (end 127.5623 103.481396) (stroke (width 0.05) (type default)) (layer "Edge.Cuts"))
 (gr_line (start 127.307227 110.482262) (end 127.120127 110.957242) (stroke (width 0.05) (type default)) (layer "Edge.Cuts"))
 (gr_line (start 127.486009 110.004089) (end 127.307227 110.482262) (stroke (width 0.05) (type default)) (layer "Edge.Cuts"))
 (gr_line (start 127.5623 103.481396) (end 127.875 103.680607) (stroke (width 0.05) (type default)) (layer "Edge.Cuts"))
 (gr_line (start 127.656418 109.522868) (end 127.486009 110.004089) (stroke (width 0.05) (type default)) (layer "Edge.Cuts"))
 (gr_line (start 127.818403 109.038747) (end 127.656418 109.522868) (stroke (width 0.05) (type default)) (layer "Edge.Cuts"))
 (gr_line (start 127.875 103.680607) (end 128.203871 103.851808) (stroke (width 0.05) (type default)) (layer "Edge.Cuts"))
 (gr_line (start 127.971914 108.551872) (end 127.818403 109.038747) (stroke (width 0.05) (type default)) (layer "Edge.Cuts"))
 (gr_line (start 128.116904 108.062392) (end 127.971914 108.551872) (stroke (width 0.05) (type default)) (layer "Edge.Cuts"))
 (gr_line (start 128.203871 103.851808) (end 128.546414 103.993693) (stroke (width 0.05) (type default)) (layer "Edge.Cuts"))
 (gr_line (start 128.25333 107.570457) (end 128.116904 108.062392) (stroke (width 0.05) (type default)) (layer "Edge.Cuts"))
 (gr_line (start 128.381149 107.076215) (end 128.25333 107.570457) (stroke (width 0.05) (type default)) (layer "Edge.Cuts"))
 (gr_line (start 128.500324 106.579818) (end 128.381149 107.076215) (stroke (width 0.05) (type default)) (layer "Edge.Cuts"))
 (gr_line (start 128.546414 103.993693) (end 128.900018 104.105184) (stroke (width 0.05) (type default)) (layer "Edge.Cuts"))
 (gr_line (start 128.610817 106.081416) (end 128.500324 106.579818) (stroke (width 0.05) (type default)) (layer "Edge.Cuts"))
 (gr_line (start 128.712595 105.581163) (end 128.610817 106.081416) (stroke (width 0.05) (type default)) (layer "Edge.Cuts"))
 (gr_line (start 128.805625 105.079209) (end 128.712595 105.581163) (stroke (width 0.05) (type default)) (layer "Edge.Cuts"))
 (gr_line (start 128.889883 104.575708) (end 128.805625 105.079209) (stroke (width 0.05) (type default)) (layer "Edge.Cuts"))
 (gr_line (start 128.900018 104.105184) (end 128.958273 104.118098) (stroke (width 0.05) (type default)) (layer "Edge.Cuts"))
 (gr_line (start 128.958273 104.118098) (end 128.889883 104.575708) (stroke (width 0.05) (type default)) (layer "Edge.Cuts"))
 (segment (start 113.48125 108.275) (end 116 108.275) (width 0.6) (layer "F.Cu") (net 1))
 (segment (start 113.2 108.61875) (end 113.2 108.55625) (width 0.6) (layer "F.Cu") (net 1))
 (segment (start 117.367098 107.6) (end 126.4 107.6) (width 0.6) (layer "F.Cu") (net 1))
 (segment (start 108.5 120.5) (end 108.5 110.1) (width 0.6) (layer "F.Cu") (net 1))
 (segment (start 109.7 108.9) (end 112.91875 108.9) (width 0.6) (layer "F.Cu") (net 1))
 (segment (start 116 108.275) (end 116.69573 107.805381) (width 0.6) (layer "F.Cu") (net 1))
 (arc (start 112.91875 108.9) (mid 113.117623 108.817623) (end 113.2 108.61875) (width 0.6) (layer "F.Cu") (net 1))
 (arc (start 116.69573 107.805381) (mid 117.016058 107.652493) (end 117.367098 107.6) (width 0.6) (layer "F.Cu") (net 1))
 (arc (start 113.2 108.55625) (mid 113.282376 108.357376) (end 113.48125 108.275) (width 0.6) (layer "F.Cu") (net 1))
 (arc (start 108.5 110.1) (mid 108.851471 109.251471) (end 109.7 108.9) (width 0.6) (layer "F.Cu") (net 1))
 (segment (start 109.325 123.04) (end 108.5 123.04) (width 0.6) (layer "F.Cu") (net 2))
 (segment (start 113.2 113.5) (end 111.2 113.5) (width 0.6) (layer "F.Cu") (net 2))
 (segment (start 110 114.7) (end 110 122.365) (width 0.6) (layer "F.Cu") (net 2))
 (segment (start 124.935362 104.8) (end 126.4 104.8) (width 0.6) (layer "F.Cu") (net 2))
 (segment (start 116 105.325) (end 124.864698 104.802082) (width 0.6) (layer "F.Cu") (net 2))
 (arc (start 110 122.365) (mid 109.802297 122.842297) (end 109.325 123.04) (width 0.6) (layer "F.Cu") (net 2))
 (arc (start 124.864698 104.802082) (mid 124.900015 104.80052) (end 124.935362 104.8) (width 0.6) (layer "F.Cu") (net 2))
 (arc (start 111.2 113.5) (mid 110.351471 113.851471) (end 110 114.7) (width 0.6) (layer "F.Cu") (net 2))
 (segment (start 108.5 123.04) (end 110.3 123.04) (width 0.6) (layer "B.Cu") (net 2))
 (segment (start 111.5 121.84) (end 111.5 104) (width 0.6) (layer "B.Cu") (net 2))
 (segment (start 112.7 102.8) (end 123.902943 102.8) (width 0.6) (layer "B.Cu") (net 2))
 (segment (start 124.751471 103.151471) (end 126.4 104.8) (width 0.6) (layer "B.Cu") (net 2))
 (arc (start 110.3 123.04) (mid 111.148528 122.688528) (end 111.5 121.84) (width 0.6) (layer "B.Cu") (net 2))
 (arc (start 123.902943 102.8) (mid 124.362163 102.891344) (end 124.751471 103.151471) (width 0.6) (layer "B.Cu") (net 2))
 (arc (start 111.5 104) (mid 111.851471 103.151471) (end 112.7 102.8) (width 0.6) (layer "B.Cu") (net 2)))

